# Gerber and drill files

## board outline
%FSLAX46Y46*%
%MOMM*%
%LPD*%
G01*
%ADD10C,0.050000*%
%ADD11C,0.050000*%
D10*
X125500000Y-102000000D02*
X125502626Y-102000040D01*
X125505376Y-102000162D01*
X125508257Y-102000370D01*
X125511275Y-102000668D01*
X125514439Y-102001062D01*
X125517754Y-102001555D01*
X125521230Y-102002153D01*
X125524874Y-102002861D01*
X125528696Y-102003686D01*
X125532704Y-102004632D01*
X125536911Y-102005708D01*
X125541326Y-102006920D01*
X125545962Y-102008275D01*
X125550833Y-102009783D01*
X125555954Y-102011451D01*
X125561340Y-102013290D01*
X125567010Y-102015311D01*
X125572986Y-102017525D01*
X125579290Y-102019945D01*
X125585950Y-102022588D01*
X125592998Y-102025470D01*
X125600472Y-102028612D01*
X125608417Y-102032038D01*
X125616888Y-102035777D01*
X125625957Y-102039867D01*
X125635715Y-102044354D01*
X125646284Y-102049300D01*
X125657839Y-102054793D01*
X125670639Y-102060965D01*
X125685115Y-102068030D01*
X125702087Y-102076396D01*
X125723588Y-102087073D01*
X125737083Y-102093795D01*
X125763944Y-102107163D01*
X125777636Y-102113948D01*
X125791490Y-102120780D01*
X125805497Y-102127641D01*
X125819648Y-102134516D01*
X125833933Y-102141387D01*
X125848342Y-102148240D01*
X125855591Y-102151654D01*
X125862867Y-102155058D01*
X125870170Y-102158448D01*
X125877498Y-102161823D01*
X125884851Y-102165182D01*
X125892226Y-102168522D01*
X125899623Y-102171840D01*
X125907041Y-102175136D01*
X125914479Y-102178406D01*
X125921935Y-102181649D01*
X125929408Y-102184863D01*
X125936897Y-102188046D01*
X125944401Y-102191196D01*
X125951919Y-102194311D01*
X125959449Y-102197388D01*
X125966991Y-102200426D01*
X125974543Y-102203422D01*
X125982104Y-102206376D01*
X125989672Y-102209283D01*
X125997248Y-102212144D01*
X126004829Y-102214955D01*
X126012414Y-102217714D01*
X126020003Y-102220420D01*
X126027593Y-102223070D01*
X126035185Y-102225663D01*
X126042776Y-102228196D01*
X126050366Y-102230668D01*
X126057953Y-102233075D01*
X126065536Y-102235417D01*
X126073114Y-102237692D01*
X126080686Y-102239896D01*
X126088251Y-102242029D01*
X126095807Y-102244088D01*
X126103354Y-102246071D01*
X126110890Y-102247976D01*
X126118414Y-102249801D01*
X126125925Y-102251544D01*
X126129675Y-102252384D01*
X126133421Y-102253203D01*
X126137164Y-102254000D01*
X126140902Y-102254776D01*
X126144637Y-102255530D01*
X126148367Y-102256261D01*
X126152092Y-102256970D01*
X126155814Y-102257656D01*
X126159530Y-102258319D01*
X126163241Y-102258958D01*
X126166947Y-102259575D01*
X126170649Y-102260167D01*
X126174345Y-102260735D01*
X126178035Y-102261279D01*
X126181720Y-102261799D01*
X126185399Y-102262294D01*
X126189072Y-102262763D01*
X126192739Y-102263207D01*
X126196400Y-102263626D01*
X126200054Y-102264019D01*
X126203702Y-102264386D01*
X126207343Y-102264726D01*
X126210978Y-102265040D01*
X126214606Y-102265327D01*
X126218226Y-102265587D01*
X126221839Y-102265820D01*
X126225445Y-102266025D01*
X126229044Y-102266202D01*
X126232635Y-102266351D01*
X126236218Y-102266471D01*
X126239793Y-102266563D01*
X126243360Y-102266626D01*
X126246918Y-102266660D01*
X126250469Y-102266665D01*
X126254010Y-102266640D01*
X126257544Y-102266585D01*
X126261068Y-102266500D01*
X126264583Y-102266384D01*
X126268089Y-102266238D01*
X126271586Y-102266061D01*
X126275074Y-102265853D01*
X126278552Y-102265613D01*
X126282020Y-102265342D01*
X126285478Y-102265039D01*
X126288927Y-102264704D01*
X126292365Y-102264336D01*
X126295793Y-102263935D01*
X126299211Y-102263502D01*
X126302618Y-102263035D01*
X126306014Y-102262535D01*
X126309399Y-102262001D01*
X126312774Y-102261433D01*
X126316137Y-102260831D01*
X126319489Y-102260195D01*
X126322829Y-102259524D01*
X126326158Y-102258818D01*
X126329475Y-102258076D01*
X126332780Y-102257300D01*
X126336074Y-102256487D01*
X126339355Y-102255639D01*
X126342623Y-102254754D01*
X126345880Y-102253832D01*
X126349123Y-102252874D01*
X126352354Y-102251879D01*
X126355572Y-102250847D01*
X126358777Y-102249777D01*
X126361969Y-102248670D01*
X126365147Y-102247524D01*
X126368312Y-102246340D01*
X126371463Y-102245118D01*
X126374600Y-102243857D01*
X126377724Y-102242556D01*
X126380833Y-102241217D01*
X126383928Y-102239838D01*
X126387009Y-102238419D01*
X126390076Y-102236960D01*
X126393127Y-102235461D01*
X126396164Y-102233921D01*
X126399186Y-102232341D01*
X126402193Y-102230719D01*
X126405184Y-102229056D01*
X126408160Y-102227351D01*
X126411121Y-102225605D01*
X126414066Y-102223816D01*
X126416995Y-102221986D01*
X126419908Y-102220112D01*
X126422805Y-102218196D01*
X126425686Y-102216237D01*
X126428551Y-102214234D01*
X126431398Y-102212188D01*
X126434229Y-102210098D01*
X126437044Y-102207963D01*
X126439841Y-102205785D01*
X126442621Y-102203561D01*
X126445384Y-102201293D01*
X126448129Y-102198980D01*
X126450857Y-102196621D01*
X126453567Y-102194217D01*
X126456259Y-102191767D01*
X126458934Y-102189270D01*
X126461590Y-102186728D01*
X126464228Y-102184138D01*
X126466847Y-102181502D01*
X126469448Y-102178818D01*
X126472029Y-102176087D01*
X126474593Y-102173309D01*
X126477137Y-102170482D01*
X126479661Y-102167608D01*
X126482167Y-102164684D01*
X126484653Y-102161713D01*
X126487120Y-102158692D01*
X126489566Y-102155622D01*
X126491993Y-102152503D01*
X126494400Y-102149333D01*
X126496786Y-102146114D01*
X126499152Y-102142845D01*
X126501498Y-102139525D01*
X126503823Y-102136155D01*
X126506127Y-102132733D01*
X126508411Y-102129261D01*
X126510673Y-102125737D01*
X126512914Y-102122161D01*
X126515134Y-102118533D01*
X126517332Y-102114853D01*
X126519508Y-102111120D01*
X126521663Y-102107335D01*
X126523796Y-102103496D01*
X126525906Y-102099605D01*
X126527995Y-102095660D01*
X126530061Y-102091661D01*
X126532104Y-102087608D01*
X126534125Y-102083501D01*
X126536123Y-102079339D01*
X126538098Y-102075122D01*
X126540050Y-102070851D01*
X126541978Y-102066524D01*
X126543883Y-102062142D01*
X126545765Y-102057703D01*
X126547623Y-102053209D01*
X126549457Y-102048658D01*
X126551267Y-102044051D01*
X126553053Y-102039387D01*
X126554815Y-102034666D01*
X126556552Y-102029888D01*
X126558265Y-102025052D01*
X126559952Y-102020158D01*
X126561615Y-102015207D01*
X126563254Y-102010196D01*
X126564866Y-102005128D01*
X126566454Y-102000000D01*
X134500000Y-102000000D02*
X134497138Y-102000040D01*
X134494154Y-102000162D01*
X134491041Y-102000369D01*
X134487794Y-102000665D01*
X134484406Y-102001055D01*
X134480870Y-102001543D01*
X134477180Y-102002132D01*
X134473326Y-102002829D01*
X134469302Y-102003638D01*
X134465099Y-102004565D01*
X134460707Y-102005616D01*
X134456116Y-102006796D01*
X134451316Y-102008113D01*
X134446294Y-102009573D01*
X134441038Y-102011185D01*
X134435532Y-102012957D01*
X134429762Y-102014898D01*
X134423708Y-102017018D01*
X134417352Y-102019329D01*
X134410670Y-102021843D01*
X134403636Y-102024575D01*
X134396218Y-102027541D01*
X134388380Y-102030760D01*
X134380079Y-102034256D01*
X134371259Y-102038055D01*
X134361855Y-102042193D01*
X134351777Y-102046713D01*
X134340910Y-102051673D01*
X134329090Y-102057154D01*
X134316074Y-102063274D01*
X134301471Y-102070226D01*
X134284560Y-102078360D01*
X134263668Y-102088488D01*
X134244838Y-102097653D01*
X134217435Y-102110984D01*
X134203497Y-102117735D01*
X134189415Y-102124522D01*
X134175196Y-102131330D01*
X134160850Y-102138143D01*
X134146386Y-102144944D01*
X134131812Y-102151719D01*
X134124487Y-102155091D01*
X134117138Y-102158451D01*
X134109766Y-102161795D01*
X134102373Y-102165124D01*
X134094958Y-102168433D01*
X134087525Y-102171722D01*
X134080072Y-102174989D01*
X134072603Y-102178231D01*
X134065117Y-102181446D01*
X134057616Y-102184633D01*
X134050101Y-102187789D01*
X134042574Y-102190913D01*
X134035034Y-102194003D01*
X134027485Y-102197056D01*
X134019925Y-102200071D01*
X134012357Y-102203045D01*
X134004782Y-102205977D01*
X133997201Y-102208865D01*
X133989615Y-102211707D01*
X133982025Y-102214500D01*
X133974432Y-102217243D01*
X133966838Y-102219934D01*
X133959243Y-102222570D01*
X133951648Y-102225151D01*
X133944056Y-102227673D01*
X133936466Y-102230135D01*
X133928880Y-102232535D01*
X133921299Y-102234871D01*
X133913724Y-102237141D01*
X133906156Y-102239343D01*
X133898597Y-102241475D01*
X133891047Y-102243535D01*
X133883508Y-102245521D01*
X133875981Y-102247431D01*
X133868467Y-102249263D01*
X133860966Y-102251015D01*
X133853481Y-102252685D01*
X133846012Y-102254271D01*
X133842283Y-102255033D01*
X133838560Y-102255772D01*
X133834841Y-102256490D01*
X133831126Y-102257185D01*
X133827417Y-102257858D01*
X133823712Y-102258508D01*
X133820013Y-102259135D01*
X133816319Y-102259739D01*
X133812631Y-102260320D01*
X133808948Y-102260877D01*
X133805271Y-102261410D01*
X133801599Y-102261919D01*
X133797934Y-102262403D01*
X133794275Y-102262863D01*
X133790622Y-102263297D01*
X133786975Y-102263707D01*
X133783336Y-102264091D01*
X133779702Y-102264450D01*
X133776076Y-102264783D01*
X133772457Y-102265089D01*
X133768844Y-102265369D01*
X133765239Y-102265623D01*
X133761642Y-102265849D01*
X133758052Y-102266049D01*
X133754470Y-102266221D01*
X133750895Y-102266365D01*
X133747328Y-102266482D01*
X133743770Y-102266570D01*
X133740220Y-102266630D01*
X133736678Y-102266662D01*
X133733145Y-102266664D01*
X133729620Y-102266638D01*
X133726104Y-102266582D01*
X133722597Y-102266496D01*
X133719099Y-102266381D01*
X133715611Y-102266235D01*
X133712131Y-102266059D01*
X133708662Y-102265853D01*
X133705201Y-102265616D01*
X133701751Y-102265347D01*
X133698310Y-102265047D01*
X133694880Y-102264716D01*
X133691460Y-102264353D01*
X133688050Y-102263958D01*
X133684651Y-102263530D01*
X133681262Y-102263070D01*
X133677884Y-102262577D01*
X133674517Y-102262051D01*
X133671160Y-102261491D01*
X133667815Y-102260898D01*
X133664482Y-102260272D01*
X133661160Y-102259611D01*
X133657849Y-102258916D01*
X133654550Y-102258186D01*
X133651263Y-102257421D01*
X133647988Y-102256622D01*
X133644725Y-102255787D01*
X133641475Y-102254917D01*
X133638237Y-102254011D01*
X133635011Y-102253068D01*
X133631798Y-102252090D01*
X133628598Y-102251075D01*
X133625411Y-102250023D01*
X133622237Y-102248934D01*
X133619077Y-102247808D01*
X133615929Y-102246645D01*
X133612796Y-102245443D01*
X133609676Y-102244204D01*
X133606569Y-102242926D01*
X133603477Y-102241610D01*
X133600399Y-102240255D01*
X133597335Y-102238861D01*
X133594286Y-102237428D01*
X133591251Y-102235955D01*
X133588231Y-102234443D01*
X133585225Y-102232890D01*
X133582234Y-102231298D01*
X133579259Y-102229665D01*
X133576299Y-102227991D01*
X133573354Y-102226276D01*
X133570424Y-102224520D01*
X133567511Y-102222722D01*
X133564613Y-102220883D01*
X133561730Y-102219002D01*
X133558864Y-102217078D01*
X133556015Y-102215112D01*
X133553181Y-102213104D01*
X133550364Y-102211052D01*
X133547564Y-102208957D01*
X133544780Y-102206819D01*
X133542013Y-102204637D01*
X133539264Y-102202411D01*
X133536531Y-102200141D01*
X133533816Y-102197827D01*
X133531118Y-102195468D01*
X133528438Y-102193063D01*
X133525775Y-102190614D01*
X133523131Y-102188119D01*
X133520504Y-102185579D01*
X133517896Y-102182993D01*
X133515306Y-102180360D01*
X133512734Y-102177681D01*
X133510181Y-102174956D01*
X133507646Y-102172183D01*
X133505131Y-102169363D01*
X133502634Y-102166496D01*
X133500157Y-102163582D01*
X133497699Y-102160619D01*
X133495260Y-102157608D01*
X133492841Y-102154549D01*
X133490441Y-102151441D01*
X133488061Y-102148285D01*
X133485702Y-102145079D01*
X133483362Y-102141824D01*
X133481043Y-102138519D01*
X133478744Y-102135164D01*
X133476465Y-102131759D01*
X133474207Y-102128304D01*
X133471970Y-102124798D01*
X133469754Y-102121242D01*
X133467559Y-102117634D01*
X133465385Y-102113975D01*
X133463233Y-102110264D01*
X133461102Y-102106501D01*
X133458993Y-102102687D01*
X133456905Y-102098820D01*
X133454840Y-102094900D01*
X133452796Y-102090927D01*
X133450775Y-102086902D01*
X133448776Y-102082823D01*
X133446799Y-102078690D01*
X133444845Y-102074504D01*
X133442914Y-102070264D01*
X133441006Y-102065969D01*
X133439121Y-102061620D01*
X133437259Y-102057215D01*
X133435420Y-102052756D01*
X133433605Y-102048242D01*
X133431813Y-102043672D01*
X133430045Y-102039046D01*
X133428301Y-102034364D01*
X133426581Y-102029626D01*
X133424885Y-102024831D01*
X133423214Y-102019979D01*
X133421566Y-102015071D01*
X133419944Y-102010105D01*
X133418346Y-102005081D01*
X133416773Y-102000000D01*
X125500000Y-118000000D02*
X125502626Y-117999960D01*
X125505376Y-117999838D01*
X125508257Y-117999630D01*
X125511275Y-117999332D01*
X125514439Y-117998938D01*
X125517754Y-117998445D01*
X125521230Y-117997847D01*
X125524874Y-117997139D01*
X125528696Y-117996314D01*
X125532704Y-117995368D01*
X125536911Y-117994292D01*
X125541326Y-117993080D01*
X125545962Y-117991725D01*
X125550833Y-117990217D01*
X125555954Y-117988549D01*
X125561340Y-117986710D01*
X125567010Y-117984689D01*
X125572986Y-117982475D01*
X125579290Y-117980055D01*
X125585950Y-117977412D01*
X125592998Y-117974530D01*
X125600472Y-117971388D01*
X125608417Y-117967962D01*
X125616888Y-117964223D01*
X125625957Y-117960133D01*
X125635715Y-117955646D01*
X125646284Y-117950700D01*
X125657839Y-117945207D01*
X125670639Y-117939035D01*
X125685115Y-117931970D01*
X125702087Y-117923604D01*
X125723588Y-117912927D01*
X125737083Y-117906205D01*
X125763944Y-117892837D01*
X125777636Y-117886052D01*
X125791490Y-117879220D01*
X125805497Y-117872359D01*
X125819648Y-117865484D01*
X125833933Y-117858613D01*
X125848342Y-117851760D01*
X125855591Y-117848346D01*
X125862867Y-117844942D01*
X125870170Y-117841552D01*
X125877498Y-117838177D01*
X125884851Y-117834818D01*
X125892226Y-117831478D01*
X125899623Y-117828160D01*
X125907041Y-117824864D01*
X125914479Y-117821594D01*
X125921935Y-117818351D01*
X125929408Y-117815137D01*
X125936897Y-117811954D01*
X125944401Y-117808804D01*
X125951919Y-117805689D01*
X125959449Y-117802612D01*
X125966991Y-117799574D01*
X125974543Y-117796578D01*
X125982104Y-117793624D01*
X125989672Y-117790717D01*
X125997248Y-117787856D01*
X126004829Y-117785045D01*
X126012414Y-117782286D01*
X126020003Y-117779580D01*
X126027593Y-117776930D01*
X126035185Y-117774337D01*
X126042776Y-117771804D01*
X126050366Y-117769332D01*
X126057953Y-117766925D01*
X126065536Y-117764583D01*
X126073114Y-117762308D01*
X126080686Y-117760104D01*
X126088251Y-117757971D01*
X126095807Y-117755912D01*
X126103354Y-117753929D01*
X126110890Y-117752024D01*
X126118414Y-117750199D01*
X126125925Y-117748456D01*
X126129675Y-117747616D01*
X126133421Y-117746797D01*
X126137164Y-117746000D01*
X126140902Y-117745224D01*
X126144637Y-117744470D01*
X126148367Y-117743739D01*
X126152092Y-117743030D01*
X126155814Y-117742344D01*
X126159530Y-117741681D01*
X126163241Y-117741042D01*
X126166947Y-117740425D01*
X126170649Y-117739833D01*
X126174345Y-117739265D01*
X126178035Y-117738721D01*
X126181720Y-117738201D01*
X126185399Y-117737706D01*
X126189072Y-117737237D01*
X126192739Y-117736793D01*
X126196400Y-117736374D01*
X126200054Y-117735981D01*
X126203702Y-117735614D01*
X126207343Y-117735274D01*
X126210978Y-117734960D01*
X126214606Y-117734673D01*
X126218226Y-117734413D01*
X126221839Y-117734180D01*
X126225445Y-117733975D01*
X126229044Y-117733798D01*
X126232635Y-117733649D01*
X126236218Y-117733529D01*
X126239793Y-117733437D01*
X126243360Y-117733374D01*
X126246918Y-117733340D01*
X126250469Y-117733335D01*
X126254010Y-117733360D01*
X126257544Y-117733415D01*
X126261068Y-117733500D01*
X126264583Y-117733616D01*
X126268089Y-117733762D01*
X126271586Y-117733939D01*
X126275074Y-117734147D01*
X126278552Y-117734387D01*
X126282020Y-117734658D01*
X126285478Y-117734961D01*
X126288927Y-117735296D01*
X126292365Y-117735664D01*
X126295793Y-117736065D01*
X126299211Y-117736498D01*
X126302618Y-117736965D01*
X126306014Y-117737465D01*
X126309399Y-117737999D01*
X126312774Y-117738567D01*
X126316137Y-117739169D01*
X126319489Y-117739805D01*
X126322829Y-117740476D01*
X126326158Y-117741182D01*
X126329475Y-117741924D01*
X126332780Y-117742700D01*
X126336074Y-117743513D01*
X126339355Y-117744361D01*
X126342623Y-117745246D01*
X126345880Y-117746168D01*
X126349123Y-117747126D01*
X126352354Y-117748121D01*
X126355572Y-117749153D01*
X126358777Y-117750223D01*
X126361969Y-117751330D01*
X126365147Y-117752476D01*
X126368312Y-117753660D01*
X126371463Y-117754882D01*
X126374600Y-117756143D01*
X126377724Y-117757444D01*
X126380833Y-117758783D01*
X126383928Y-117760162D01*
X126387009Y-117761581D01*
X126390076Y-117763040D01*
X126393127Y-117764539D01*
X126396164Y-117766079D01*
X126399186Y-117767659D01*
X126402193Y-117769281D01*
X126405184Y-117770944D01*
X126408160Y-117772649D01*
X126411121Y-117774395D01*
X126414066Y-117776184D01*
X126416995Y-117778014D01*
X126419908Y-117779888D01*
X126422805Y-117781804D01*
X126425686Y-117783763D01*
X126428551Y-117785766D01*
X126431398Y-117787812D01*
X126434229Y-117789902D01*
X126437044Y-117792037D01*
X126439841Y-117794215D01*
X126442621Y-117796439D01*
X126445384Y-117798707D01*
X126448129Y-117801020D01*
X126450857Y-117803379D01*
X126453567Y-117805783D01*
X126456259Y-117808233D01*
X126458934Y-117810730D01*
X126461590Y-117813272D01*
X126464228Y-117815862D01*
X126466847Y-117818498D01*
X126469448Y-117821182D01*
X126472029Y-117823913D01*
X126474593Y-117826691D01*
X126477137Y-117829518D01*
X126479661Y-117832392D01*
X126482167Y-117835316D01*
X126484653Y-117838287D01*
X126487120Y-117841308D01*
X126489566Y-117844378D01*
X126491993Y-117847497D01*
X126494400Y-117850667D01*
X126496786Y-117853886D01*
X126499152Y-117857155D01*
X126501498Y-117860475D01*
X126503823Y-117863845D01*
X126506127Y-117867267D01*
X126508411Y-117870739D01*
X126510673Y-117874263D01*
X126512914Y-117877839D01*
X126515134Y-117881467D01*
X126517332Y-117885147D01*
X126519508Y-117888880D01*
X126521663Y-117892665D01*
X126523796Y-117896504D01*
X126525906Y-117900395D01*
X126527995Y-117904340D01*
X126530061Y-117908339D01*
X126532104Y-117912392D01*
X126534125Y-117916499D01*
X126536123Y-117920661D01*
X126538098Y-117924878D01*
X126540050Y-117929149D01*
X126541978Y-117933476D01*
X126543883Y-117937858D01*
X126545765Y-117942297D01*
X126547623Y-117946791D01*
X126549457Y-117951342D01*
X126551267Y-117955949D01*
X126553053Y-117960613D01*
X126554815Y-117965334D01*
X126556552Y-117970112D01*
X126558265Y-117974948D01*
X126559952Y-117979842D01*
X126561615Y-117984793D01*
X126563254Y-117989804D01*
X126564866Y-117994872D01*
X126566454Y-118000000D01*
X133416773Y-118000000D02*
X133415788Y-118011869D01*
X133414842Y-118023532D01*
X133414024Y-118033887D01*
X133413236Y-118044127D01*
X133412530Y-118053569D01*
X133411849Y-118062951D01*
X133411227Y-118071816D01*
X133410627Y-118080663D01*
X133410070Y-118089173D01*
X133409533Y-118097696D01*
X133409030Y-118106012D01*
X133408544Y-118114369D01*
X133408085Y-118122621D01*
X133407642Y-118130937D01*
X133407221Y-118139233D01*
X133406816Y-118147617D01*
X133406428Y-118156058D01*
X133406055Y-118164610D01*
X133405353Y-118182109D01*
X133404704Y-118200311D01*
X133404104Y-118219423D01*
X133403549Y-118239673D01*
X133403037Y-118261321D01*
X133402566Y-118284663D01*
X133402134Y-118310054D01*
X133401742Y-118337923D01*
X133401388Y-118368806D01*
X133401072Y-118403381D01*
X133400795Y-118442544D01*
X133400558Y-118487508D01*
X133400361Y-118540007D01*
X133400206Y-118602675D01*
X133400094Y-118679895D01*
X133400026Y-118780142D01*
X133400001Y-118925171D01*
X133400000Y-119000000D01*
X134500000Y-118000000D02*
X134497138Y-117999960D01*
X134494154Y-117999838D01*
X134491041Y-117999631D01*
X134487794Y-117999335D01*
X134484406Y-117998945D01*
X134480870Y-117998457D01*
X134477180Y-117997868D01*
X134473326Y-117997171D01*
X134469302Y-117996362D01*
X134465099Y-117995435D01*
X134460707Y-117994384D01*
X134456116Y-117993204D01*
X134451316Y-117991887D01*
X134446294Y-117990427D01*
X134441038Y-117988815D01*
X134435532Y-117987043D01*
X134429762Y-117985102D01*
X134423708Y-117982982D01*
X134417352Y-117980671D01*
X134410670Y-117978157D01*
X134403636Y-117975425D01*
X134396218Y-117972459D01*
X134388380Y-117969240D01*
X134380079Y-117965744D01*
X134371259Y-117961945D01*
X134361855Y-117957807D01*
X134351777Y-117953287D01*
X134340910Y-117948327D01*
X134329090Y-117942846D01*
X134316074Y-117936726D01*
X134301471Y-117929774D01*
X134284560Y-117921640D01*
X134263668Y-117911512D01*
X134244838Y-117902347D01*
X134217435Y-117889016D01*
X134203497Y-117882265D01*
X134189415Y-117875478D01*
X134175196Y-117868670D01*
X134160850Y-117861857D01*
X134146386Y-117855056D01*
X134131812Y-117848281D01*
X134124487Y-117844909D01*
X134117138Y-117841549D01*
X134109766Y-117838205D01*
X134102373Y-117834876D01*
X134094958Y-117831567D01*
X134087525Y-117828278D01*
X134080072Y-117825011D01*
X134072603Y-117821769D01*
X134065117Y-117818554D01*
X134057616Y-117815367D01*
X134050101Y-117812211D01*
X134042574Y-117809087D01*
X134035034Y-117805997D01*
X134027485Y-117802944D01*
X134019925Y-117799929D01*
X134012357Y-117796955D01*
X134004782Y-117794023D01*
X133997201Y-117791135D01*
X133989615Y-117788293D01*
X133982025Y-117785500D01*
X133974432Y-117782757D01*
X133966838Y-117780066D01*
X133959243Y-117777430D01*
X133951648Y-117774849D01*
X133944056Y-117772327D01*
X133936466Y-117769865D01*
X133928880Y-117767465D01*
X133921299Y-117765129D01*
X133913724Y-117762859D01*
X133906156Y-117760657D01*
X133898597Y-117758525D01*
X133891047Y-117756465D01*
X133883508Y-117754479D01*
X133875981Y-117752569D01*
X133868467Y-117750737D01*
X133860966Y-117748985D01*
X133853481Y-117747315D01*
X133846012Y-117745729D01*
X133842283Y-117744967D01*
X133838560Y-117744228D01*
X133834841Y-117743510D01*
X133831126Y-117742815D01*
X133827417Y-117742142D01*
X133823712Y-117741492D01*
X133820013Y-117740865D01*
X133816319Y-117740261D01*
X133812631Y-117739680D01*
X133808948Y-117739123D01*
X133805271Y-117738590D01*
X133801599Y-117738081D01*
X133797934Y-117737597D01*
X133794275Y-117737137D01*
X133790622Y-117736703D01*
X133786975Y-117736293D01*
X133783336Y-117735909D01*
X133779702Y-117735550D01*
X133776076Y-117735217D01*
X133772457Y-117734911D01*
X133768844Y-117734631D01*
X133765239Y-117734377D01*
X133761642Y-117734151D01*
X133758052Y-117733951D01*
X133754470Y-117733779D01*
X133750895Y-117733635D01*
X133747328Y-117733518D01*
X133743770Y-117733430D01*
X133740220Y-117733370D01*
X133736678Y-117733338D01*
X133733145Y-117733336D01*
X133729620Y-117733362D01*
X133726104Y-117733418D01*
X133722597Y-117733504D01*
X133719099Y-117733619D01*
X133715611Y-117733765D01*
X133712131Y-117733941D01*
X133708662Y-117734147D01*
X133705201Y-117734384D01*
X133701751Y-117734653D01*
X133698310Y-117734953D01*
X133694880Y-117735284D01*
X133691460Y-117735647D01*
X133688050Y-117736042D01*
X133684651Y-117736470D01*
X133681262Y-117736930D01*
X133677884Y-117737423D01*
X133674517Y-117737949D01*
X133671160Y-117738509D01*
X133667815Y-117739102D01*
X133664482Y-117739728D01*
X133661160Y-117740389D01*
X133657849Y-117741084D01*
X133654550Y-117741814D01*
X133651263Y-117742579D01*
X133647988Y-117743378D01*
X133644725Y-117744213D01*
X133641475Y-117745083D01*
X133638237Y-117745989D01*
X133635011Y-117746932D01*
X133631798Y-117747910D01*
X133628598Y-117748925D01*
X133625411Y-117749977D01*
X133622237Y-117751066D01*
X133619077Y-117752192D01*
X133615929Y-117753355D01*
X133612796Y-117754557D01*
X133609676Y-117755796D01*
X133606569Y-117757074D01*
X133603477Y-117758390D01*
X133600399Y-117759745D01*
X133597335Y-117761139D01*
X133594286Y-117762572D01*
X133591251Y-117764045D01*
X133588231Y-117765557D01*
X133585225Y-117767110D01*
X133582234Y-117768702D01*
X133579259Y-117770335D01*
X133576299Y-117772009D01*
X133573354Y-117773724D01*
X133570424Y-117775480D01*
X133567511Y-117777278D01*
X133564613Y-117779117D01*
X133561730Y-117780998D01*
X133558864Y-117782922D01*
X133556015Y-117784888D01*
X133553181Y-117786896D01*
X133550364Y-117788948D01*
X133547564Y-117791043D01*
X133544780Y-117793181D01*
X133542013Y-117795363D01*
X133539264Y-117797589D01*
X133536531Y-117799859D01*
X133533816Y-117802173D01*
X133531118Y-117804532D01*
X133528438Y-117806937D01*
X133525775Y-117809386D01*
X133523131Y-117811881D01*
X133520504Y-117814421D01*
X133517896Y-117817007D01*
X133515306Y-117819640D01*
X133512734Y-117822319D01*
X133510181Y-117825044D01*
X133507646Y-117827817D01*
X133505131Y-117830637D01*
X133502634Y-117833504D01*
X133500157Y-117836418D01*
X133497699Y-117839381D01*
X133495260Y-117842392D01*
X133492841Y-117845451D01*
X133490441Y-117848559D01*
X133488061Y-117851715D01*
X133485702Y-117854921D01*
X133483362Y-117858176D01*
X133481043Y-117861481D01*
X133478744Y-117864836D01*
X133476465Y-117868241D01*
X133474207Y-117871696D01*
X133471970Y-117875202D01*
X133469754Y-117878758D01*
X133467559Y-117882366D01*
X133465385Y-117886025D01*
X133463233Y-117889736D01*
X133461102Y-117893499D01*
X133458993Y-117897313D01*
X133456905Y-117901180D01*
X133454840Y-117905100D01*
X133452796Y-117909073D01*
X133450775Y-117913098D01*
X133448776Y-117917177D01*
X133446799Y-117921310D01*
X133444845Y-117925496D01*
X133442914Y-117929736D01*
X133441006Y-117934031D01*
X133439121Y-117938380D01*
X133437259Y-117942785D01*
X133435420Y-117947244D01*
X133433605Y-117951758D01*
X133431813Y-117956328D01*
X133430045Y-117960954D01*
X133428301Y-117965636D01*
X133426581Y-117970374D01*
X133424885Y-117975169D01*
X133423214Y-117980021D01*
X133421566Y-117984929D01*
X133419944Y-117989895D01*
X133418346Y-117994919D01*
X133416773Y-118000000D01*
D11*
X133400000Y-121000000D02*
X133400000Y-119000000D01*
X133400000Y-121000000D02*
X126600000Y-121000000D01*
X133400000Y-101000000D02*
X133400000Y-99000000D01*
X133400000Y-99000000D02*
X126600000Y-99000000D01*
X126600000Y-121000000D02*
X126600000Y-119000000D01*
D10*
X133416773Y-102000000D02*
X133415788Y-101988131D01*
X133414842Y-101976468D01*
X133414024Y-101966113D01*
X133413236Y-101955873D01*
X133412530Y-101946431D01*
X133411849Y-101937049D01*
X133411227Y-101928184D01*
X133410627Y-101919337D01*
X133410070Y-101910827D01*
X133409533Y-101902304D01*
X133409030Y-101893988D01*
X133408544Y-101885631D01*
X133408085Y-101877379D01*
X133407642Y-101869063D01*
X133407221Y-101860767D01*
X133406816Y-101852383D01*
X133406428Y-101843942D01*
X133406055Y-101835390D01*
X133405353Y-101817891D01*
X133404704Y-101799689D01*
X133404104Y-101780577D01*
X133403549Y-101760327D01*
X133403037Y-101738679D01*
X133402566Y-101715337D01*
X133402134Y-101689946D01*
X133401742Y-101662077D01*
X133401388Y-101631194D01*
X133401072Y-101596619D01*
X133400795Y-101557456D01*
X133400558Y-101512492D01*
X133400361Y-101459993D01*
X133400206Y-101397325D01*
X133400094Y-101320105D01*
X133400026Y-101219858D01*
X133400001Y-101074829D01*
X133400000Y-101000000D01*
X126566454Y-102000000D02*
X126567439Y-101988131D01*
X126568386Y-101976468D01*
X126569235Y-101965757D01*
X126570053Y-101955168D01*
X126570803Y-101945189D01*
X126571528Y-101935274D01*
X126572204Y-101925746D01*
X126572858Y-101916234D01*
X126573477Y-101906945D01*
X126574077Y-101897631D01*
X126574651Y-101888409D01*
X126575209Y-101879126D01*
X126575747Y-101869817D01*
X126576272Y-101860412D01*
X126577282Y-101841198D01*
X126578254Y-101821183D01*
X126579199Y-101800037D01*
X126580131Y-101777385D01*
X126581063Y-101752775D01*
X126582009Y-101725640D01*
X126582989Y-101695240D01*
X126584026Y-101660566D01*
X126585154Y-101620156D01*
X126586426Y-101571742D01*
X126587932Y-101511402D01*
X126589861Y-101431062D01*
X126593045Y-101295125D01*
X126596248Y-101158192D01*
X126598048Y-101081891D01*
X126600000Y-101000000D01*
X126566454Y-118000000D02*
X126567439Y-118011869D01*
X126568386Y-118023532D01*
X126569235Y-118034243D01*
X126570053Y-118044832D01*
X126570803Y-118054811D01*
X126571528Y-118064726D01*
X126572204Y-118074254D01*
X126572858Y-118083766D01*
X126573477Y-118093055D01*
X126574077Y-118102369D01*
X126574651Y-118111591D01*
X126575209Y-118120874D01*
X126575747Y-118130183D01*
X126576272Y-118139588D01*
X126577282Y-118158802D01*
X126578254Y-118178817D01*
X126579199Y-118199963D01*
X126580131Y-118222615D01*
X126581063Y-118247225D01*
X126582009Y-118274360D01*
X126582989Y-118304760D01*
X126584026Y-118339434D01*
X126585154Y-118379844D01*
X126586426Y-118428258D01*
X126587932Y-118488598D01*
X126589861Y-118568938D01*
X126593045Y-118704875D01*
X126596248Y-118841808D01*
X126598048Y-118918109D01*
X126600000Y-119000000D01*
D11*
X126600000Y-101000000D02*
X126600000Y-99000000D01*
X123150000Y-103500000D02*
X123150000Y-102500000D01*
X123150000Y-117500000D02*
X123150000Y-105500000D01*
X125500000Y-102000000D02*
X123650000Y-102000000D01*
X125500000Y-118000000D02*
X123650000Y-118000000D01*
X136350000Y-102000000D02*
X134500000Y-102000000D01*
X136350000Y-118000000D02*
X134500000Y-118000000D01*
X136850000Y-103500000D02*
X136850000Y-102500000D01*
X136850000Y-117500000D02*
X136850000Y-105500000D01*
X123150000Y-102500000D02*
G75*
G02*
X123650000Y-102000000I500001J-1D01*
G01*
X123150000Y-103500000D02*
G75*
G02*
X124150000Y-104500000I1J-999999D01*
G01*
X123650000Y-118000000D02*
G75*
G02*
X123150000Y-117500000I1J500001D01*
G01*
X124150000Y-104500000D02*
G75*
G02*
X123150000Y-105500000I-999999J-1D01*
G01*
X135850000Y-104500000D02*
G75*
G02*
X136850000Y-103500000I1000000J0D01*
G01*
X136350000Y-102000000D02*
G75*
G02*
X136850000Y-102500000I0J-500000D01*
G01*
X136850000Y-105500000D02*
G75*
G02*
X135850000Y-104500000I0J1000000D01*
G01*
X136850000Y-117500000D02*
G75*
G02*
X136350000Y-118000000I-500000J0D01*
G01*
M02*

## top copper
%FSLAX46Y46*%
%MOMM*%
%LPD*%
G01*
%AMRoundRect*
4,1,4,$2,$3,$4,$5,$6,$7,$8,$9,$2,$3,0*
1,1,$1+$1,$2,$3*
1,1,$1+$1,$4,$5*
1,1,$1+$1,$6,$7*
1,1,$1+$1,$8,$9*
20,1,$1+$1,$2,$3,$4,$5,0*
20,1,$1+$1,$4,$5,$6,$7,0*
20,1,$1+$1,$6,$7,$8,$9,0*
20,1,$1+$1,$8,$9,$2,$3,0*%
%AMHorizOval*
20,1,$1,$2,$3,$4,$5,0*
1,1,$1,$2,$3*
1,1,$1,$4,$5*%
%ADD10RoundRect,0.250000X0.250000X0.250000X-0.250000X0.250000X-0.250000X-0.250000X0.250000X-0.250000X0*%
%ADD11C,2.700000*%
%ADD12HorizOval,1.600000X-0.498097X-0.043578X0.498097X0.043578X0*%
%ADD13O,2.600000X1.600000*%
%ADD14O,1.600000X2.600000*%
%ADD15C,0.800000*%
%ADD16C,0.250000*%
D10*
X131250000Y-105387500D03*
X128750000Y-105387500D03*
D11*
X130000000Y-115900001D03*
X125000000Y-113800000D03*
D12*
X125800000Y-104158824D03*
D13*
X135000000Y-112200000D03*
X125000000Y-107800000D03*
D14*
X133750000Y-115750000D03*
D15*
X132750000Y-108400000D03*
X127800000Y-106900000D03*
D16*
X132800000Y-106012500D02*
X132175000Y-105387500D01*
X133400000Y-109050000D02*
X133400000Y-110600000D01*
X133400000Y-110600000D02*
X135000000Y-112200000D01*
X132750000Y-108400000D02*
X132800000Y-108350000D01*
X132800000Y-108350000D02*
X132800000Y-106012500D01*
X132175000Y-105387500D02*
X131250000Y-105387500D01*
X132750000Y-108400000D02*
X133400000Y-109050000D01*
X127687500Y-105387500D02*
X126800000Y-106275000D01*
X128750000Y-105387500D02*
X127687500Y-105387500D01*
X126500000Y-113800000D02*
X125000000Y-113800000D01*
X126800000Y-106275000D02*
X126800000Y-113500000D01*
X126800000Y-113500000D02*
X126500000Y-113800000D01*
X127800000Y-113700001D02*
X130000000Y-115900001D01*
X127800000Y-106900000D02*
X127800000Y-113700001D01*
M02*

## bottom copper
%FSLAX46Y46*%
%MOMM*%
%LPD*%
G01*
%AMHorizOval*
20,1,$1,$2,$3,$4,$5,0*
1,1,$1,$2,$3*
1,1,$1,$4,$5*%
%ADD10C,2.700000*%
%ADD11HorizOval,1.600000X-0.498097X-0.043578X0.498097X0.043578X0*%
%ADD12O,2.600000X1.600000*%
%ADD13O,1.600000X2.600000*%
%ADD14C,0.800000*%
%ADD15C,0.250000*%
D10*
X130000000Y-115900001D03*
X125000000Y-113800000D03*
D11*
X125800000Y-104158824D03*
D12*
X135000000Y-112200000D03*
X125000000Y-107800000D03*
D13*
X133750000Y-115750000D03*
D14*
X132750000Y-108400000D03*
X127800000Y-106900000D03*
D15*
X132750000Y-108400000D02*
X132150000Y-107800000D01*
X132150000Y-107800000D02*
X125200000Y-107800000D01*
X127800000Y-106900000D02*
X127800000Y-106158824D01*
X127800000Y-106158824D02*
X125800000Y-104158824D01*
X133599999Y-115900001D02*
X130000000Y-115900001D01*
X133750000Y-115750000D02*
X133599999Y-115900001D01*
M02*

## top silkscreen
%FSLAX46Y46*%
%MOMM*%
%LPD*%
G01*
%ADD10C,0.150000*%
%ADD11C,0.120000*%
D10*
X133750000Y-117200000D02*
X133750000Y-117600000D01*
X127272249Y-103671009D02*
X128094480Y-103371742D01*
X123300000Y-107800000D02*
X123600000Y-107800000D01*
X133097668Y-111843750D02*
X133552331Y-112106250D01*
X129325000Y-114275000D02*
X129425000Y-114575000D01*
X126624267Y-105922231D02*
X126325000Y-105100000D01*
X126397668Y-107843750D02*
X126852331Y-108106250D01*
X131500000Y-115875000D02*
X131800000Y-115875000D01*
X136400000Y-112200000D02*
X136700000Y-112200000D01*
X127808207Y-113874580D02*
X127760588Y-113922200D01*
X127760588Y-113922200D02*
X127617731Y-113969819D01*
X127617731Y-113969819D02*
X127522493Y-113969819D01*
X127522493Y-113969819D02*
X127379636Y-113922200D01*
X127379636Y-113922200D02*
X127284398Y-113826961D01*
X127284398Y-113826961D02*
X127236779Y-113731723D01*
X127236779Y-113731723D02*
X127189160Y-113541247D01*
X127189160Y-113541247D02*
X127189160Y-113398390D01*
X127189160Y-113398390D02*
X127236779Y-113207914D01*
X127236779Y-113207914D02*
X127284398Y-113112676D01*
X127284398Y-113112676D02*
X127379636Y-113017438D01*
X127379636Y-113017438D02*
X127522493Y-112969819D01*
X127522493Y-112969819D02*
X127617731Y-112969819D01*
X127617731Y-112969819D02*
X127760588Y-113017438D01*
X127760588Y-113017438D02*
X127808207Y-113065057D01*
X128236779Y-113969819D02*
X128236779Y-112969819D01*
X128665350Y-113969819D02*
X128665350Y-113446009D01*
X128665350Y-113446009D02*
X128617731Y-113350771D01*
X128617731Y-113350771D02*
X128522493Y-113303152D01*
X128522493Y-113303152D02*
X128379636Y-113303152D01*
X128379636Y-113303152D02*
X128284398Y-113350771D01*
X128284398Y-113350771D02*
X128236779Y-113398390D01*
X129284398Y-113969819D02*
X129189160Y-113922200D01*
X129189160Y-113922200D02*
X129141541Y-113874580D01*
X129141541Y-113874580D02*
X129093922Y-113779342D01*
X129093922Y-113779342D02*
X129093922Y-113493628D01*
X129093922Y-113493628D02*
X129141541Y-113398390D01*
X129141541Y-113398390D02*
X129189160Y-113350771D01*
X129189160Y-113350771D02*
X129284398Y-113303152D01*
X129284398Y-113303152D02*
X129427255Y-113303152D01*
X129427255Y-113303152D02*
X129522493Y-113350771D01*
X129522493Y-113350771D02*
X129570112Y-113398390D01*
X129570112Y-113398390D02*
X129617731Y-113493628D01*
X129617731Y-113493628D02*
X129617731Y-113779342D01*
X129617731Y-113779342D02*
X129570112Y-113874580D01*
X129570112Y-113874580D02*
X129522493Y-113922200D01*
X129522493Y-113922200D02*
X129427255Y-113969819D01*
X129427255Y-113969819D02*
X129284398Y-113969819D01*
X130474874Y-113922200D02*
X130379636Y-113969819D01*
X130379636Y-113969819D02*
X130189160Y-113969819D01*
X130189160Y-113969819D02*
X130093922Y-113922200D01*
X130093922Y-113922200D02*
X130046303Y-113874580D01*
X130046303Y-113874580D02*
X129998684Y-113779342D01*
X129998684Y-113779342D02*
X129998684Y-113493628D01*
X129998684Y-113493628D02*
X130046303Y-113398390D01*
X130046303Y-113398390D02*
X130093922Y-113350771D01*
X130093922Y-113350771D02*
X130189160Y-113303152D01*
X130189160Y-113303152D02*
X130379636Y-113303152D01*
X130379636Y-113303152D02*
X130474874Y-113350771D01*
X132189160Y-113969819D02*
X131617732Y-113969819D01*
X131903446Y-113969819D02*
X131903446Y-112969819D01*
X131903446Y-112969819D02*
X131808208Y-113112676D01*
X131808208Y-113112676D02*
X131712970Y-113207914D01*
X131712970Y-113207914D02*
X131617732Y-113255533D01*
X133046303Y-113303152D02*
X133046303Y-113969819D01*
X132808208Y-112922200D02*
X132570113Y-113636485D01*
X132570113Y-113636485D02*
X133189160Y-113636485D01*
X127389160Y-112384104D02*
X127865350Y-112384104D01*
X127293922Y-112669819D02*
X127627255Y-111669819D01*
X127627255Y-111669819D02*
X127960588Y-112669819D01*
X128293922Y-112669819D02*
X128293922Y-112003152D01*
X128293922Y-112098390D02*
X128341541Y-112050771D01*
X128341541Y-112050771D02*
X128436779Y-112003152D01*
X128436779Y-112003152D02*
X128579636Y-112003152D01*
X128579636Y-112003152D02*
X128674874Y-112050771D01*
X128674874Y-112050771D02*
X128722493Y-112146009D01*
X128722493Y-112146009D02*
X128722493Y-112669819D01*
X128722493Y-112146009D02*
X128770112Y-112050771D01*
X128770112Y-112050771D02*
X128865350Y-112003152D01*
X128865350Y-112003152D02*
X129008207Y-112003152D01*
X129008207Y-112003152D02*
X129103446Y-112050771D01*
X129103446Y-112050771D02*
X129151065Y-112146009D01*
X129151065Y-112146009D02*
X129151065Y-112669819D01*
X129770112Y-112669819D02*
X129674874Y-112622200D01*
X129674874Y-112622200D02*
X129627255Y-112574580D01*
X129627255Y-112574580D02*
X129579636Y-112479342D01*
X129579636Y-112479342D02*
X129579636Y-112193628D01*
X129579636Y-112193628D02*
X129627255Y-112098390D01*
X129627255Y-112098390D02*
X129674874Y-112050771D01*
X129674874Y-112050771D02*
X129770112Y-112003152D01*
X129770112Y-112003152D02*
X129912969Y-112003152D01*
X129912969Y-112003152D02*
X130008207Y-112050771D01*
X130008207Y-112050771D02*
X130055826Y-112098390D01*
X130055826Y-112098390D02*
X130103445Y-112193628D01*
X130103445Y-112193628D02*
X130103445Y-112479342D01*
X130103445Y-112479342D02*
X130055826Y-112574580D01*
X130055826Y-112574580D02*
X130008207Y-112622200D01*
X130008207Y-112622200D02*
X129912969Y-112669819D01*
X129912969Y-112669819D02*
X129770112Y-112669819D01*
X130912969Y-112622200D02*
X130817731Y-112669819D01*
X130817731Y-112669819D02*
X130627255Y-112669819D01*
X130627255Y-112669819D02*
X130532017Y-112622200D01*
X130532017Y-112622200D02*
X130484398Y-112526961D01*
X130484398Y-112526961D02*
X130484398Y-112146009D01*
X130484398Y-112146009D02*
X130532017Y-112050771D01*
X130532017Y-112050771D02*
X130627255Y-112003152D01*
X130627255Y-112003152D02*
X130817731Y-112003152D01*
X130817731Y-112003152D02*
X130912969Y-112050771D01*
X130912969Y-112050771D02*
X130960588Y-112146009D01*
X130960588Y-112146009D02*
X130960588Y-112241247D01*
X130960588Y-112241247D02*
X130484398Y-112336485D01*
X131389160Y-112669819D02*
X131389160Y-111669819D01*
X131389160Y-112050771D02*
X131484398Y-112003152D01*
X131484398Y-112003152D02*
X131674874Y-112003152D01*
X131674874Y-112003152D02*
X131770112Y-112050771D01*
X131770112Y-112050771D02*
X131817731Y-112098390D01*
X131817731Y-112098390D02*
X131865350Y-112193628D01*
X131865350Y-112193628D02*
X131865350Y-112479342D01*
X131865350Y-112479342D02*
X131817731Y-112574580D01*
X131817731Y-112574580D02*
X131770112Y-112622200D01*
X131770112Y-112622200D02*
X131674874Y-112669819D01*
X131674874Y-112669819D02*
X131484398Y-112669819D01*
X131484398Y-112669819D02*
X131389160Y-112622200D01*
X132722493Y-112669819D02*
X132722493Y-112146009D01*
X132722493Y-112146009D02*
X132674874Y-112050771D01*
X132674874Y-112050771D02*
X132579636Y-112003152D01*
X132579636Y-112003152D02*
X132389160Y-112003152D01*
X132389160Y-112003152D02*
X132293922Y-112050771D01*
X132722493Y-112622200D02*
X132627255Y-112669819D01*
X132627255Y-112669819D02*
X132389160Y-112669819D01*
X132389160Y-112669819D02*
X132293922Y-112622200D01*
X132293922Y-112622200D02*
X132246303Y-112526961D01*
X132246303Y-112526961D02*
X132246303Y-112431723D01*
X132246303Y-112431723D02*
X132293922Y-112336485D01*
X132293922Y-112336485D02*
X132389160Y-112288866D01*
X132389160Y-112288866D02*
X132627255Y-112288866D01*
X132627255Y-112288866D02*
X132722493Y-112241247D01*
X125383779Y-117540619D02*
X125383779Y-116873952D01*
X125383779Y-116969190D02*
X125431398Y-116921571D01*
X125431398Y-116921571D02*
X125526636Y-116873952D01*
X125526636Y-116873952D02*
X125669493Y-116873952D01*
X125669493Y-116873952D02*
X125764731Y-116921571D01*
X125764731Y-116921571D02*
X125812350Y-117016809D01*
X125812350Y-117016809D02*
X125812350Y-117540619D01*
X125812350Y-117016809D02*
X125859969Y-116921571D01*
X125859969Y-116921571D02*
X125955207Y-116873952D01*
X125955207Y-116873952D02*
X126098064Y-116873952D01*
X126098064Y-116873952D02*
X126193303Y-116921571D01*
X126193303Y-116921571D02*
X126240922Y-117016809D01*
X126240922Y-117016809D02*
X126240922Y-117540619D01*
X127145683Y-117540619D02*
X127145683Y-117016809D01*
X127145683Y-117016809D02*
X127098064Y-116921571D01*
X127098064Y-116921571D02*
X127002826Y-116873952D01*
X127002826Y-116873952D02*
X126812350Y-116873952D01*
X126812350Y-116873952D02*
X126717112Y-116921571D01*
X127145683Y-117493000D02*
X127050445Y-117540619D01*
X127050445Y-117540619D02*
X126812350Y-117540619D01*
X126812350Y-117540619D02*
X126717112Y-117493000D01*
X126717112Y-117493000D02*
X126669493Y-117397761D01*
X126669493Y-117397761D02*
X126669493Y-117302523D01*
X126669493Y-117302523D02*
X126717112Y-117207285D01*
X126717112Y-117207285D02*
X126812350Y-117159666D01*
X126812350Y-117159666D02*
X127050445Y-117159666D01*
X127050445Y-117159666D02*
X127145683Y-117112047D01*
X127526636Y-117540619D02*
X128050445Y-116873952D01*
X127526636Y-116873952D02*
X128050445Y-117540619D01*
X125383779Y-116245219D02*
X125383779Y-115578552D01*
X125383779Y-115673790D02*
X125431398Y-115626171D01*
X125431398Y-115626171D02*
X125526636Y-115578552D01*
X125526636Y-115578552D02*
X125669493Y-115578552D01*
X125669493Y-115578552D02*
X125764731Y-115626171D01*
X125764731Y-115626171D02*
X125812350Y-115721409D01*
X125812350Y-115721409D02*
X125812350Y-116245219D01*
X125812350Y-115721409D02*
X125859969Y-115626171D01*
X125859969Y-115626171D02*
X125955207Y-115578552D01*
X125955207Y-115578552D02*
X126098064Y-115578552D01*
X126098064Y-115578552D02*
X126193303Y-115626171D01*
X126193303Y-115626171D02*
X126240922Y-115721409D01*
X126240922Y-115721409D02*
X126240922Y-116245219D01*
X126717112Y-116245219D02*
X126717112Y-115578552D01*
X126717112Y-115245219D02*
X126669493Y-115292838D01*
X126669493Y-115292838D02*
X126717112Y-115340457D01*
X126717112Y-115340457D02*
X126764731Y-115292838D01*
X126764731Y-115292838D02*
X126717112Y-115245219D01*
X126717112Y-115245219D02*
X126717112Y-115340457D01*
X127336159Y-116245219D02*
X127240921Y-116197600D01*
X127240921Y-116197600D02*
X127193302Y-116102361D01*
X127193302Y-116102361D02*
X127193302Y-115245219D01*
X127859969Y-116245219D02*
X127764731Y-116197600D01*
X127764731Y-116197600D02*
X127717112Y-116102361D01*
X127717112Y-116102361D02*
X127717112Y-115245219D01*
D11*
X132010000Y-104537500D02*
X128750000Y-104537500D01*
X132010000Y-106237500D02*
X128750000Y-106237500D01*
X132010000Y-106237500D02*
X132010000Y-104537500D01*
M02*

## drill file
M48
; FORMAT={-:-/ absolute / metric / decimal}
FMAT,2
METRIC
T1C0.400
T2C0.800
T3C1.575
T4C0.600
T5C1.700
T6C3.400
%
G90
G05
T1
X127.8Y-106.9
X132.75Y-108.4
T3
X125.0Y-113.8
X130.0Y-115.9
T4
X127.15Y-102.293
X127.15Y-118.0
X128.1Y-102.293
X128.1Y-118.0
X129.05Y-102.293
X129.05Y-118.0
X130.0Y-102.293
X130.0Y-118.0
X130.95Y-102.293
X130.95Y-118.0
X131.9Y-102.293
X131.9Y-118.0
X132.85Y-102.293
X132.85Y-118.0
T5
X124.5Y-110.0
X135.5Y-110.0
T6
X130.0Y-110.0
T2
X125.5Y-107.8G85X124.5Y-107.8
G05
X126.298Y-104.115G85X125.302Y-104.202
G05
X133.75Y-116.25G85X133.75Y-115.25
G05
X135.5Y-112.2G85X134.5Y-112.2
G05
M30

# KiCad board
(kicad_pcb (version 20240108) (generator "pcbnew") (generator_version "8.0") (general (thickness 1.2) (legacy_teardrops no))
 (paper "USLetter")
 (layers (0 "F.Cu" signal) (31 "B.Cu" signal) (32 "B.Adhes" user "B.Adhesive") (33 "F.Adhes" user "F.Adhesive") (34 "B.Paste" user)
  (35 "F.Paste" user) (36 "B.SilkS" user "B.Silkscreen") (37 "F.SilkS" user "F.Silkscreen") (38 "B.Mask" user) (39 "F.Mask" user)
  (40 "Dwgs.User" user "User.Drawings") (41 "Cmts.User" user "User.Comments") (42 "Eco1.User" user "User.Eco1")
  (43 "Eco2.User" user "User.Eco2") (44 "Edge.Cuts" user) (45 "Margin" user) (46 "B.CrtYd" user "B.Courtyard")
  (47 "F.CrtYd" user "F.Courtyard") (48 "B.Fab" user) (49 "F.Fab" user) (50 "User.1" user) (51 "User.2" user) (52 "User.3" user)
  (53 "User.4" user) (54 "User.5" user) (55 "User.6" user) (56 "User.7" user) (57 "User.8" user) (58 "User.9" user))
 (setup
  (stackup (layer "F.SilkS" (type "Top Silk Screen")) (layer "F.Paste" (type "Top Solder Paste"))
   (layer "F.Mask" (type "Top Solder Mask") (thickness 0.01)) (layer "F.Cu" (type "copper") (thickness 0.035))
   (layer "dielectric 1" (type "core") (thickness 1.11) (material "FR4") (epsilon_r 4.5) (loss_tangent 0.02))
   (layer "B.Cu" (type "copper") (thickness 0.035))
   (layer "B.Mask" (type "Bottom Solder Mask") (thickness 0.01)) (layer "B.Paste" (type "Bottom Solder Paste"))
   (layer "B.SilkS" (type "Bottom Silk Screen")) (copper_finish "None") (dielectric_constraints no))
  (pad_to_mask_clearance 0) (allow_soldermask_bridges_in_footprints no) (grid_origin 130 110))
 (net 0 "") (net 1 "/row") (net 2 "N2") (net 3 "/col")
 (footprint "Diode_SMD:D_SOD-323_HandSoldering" (layer "F.Cu") (at 130 105.3875 180)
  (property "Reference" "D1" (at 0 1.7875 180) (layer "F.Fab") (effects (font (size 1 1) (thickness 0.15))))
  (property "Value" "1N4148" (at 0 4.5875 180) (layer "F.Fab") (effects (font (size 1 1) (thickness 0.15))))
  (fp_line (start -2.01 0.85) (end 1.25 0.85) (stroke (width 0.12) (type solid)) (layer "F.SilkS"))
  (fp_line (start -2.01 -0.85) (end 1.25 -0.85) (stroke (width 0.12) (type solid)) (layer "F.SilkS"))
  (fp_line (start -2.01 -0.85) (end -2.01 0.85) (stroke (width 0.12) (type solid)) (layer "F.SilkS"))
  (pad "1" smd roundrect (at -1.25 0 180) (size 1 1) (layers "F.Cu" "F.Paste" "F.Mask") (roundrect_rratio 0.25) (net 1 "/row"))
  (pad "2" smd roundrect (at 1.25 0 180) (size 1 1) (layers "F.Cu" "F.Paste" "F.Mask") (roundrect_rratio 0.25) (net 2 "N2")))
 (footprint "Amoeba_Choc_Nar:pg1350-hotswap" (layer "F.Cu") (at 130 110)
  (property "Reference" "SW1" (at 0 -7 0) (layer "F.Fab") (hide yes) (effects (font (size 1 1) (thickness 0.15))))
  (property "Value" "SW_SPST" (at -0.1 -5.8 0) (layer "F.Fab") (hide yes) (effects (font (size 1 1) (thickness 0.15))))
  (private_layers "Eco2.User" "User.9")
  (fp_line (start -6.85 -6.5) (end -6.85 -7.5) (stroke (width 0.05) (type solid)) (layer "Edge.Cuts"))
  (fp_line (start -6.85 7.5) (end -6.85 -4.5) (stroke (width 0.05) (type solid)) (layer "Edge.Cuts"))
  (fp_line (start -4.5 -8) (end -6.35 -8) (stroke (width 0.05) (type solid)) (layer "Edge.Cuts"))
  (fp_line (start -4.5 8) (end -6.35 8) (stroke (width 0.05) (type solid)) (layer "Edge.Cuts"))
  (fp_line (start 6.35 -8) (end 4.5 -8) (stroke (width 0.05) (type solid)) (layer "Edge.Cuts"))
  (fp_line (start 6.35 8) (end 4.5 8) (stroke (width 0.05) (type solid)) (layer "Edge.Cuts"))
  (fp_line (start 6.85 -6.5) (end 6.85 -7.5) (stroke (width 0.05) (type solid)) (layer "Edge.Cuts"))
  (fp_line (start 6.85 7.5) (end 6.85 -4.5) (stroke (width 0.05) (type solid)) (layer "Edge.Cuts"))
  (fp_arc (start -6.85 -7.5) (mid -6.703553 -7.853553) (end -6.35 -8) (stroke (width 0.05) (type default)) (layer "Edge.Cuts"))
  (fp_arc (start -6.85 -6.5) (mid -6.142893 -6.207107) (end -5.85 -5.5) (stroke (width 0.05) (type default)) (layer "Edge.Cuts"))
  (fp_arc (start -6.35 8) (mid -6.703553 7.853553) (end -6.85 7.5) (stroke (width 0.05) (type default)) (layer "Edge.Cuts"))
  (fp_arc (start -5.85 -5.5) (mid -6.142893 -4.792893) (end -6.85 -4.5) (stroke (width 0.05) (type default)) (layer "Edge.Cuts"))
  (fp_arc (start 5.85 -5.5) (mid 6.142893 -6.207107) (end 6.85 -6.5) (stroke (width 0.05) (type default)) (layer "Edge.Cuts"))
  (fp_arc (start 6.35 -8) (mid 6.703553 -7.853553) (end 6.85 -7.5) (stroke (width 0.05) (type default)) (layer "Edge.Cuts"))
  (fp_arc (start 6.85 -4.5) (mid 6.142893 -4.792893) (end 5.85 -5.5) (stroke (width 0.05) (type default)) (layer "Edge.Cuts"))
  (fp_arc (start 6.85 7.5) (mid 6.703553 7.853553) (end 6.35 8) (stroke (width 0.05) (type default)) (layer "Edge.Cuts"))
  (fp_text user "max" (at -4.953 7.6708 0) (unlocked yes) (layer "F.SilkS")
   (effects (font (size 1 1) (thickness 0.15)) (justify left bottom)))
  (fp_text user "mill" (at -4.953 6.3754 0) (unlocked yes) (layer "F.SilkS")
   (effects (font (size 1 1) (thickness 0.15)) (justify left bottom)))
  (pad "" np_thru_hole circle (at -5.5 0 180) (size 1.7 1.7) (drill 1.7) (layers "*.Cu" "*.Mask"))
  (pad "" np_thru_hole circle (at 0 0 180) (size 3.4 3.4) (drill 3.4) (layers "*.Cu" "*.Mask"))
  (pad "" np_thru_hole circle (at 5.5 0 180) (size 1.7 1.7) (drill 1.7) (layers "*.Cu" "*.Mask"))
  (pad "1" thru_hole circle (at 0 5.900001 180) (size 2.7 2.7) (drill 1.5748) (layers "*.Cu" "*.Mask") (remove_unused_layers no)
   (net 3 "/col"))
  (pad "2" thru_hole circle (at -5 3.8 180) (size 2.7 2.7) (drill 1.5748) (layers "*.Cu" "*.Mask") (remove_unused_layers no) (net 2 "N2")))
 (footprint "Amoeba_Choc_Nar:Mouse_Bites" (layer "F.Cu") (at 130 118)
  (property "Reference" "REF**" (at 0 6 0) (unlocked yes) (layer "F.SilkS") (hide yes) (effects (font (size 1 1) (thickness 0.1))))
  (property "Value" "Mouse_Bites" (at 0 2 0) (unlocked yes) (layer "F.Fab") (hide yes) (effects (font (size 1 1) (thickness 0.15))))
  (pad "" np_thru_hole circle (at -2.85 0) (size 0.6 0.6) (drill 0.6) (layers "*.Mask"))
  (pad "" np_thru_hole circle (at -1.9 0) (size 0.6 0.6) (drill 0.6) (layers "*.Mask"))
  (pad "" np_thru_hole circle (at -0.95 0) (size 0.6 0.6) (drill 0.6) (layers "*.Mask"))
  (pad "" np_thru_hole circle (at 0 0) (size 0.6 0.6) (drill 0.6) (layers "*.Mask"))
  (pad "" np_thru_hole circle (at 0.95 0) (size 0.6 0.6) (drill 0.6) (layers "*.Mask"))
  (pad "" np_thru_hole circle (at 1.9 0) (size 0.6 0.6) (drill 0.6) (layers "*.Mask"))
  (pad "" np_thru_hole circle (at 2.85 0) (size 0.6 0.6) (drill 0.6) (layers "*.Mask")))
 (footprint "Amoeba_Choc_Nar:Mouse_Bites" (layer "F.Cu") (at 130 102.292893)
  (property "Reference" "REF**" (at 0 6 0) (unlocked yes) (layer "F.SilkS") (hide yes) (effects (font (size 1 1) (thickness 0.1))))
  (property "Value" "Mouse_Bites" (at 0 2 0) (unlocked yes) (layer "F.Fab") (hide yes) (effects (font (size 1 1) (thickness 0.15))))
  (pad "" np_thru_hole circle (at -2.85 0) (size 0.6 0.6) (drill 0.6) (layers "*.Mask"))
  (pad "" np_thru_hole circle (at -1.9 0) (size 0.6 0.6) (drill 0.6) (layers "*.Mask"))
  (pad "" np_thru_hole circle (at -0.95 0) (size 0.6 0.6) (drill 0.6) (layers "*.Mask"))
  (pad "" np_thru_hole circle (at 0 0) (size 0.6 0.6) (drill 0.6) (layers "*.Mask"))
  (pad "" np_thru_hole circle (at 0.95 0) (size 0.6 0.6) (drill 0.6) (layers "*.Mask"))
  (pad "" np_thru_hole circle (at 1.9 0) (size 0.6 0.6) (drill 0.6) (layers "*.Mask"))
  (pad "" np_thru_hole circle (at 2.85 0) (size 0.6 0.6) (drill 0.6) (layers "*.Mask")))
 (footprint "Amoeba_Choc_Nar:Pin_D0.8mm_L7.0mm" (layer "B.Cu") (at 125.8 104.158824 -85)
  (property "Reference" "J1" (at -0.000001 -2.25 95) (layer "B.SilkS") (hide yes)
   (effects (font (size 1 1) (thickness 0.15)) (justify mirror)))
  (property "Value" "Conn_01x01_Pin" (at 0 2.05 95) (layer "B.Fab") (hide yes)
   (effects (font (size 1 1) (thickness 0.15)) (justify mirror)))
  (pad "1" thru_hole oval (at 0 0 275) (size 1.6 2.6) (drill oval 0.8 1.8) (layers "*.Cu" "*.Mask") (remove_unused_layers no) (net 3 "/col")))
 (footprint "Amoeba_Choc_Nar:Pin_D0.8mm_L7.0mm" (layer "B.Cu") (at 135 112.2 -90)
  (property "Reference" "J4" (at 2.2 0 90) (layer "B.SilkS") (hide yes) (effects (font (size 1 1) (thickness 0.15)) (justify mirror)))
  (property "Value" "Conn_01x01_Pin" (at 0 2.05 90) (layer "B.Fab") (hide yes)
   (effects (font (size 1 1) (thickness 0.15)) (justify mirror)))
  (pad "1" thru_hole oval (at 0 0 270) (size 1.6 2.6) (drill oval 0.8 1.8) (layers "*.Cu" "*.Mask") (remove_unused_layers no) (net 1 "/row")))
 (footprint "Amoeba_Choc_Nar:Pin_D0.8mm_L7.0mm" (layer "B.Cu") (at 125 107.8 -90)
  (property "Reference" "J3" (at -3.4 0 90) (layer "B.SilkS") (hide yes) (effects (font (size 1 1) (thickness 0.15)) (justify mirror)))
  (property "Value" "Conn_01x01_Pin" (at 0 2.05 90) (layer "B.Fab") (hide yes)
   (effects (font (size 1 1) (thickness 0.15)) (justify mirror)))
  (pad "1" thru_hole oval (at 0 0 270) (size 1.6 2.6) (drill oval 0.8 1.8) (layers "*.Cu" "*.Mask") (remove_unused_layers no) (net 1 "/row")))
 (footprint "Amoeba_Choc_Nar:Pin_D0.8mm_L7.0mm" (layer "B.Cu") (at 133.75 115.75 180)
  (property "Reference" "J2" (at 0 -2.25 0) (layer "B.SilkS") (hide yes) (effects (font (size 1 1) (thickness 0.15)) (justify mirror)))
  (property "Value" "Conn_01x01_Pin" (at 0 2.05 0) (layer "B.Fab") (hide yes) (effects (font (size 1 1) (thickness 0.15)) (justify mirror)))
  (pad "1" thru_hole oval (at 0 0 180) (size 1.6 2.6) (drill oval 0.8 1.8) (layers "*.Cu" "*.Mask") (remove_unused_layers no) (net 3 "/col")))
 (gr_line (start 133.75 117.2) (end 133.75 117.6) (stroke (width 0.15) (type default)) (layer "F.SilkS"))
 (gr_line (start 127.272249 103.671009) (end 128.09448 103.371742) (stroke (width 0.15) (type default)) (layer "F.SilkS"))
 (gr_line (start 123.3 107.8) (end 123.6 107.8) (stroke (width 0.15) (type default)) (layer "F.SilkS"))
 (gr_line (start 133.097668 111.84375) (end 133.552331 112.10625) (stroke (width 0.15) (type default)) (layer "F.SilkS"))
 (gr_line (start 129.325 114.275) (end 129.425 114.575) (stroke (width 0.15) (type default)) (layer "F.SilkS"))
 (gr_line (start 126.624267 105.922231) (end 126.325 105.1) (stroke (width 0.15) (type default)) (layer "F.SilkS"))
 (gr_line (start 126.397668 107.84375) (end 126.852331 108.10625) (stroke (width 0.15) (type default)) (layer "F.SilkS"))
 (gr_line (start 131.5 115.875) (end 131.8 115.875) (stroke (width 0.15) (type default)) (layer "F.SilkS"))
 (gr_line (start 136.4 112.2) (end 136.7 112.2) (stroke (width 0.15) (type default)) (layer "F.SilkS"))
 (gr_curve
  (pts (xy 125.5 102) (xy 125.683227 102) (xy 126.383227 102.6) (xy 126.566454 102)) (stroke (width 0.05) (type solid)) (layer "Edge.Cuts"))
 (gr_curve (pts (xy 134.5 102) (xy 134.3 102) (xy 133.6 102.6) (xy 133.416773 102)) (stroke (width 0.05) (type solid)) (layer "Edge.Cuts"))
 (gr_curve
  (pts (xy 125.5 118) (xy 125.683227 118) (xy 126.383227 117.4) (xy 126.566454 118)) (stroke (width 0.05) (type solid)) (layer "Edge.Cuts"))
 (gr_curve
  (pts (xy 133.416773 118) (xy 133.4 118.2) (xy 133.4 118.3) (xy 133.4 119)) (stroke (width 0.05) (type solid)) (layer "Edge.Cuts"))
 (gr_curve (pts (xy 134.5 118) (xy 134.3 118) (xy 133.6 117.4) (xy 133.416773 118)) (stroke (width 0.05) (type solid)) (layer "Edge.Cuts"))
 (gr_line (start 133.4 121) (end 133.4 119) (stroke (width 0.05) (type default)) (layer "Edge.Cuts"))
 (gr_line (start 133.4 121) (end 126.6 121) (stroke (width 0.05) (type default)) (layer "Edge.Cuts"))
 (gr_line (start 133.4 101) (end 133.4 99) (stroke (width 0.05) (type default)) (layer "Edge.Cuts"))
 (gr_line (start 133.4 99) (end 126.6 99) (stroke (width 0.05) (type default)) (layer "Edge.Cuts"))
 (gr_line (start 126.6 121) (end 126.6 119) (stroke (width 0.05) (type default)) (layer "Edge.Cuts"))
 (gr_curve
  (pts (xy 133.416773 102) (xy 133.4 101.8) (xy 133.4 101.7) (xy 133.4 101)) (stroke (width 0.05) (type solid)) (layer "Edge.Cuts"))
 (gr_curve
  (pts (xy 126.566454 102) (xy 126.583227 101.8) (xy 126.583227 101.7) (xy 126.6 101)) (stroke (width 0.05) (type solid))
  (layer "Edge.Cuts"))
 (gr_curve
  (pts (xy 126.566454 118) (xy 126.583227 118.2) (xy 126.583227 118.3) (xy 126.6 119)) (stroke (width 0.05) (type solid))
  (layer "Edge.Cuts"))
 (gr_line (start 126.6 101) (end 126.6 99) (stroke (width 0.05) (type default)) (layer "Edge.Cuts"))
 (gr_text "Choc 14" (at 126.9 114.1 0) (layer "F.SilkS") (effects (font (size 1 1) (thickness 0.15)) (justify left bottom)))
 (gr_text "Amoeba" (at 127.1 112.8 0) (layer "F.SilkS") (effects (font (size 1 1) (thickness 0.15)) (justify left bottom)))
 (segment (start 132.8 106.0125) (end 132.175 105.3875) (width 0.25) (layer "F.Cu") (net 1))
 (segment (start 133.4 109.05) (end 133.4 110.6) (width 0.25) (layer "F.Cu") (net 1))
 (segment (start 133.4 110.6) (end 135 112.2) (width 0.25) (layer "F.Cu") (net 1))
 (segment (start 132.75 108.4) (end 132.8 108.35) (width 0.25) (layer "F.Cu") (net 1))
 (segment (start 132.8 108.35) (end 132.8 106.0125) (width 0.25) (layer "F.Cu") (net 1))
 (segment (start 132.175 105.3875) (end 131.25 105.3875) (width 0.25) (layer "F.Cu") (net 1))
 (segment (start 132.75 108.4) (end 133.4 109.05) (width 0.25) (layer "F.Cu") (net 1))
 (via (at 132.75 108.4) (size 0.8) (drill 0.4) (layers "F.Cu" "B.Cu") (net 1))
 (segment (start 132.75 108.4) (end 132.15 107.8) (width 0.25) (layer "B.Cu") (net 1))
 (segment (start 132.15 107.8) (end 125.2 107.8) (width 0.25) (layer "B.Cu") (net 1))
 (segment (start 127.6875 105.3875) (end 126.8 106.275) (width 0.25) (layer "F.Cu") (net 2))
 (segment (start 128.75 105.3875) (end 127.6875 105.3875) (width 0.25) (layer "F.Cu") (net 2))
 (segment (start 126.5 113.8) (end 125 113.8) (width 0.25) (layer "F.Cu") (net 2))
 (segment (start 126.8 106.275) (end 126.8 113.5) (width 0.25) (layer "F.Cu") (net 2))
 (segment (start 126.8 113.5) (end 126.5 113.8) (width 0.25) (layer "F.Cu") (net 2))
 (segment (start 127.8 113.700001) (end 130 115.900001) (width 0.25) (layer "F.Cu") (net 3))
 (segment (start 127.8 106.9) (end 127.8 113.700001) (width 0.25) (layer "F.Cu") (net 3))
 (via (at 127.8 106.9) (size 0.8) (drill 0.4) (layers "F.Cu" "B.Cu") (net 3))
 (segment (start 127.8 106.9) (end 127.8 106.158824) (width 0.25) (layer "B.Cu") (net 3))
 (segment (start 127.8 106.158824) (end 125.8 104.158824) (width 0.25) (layer "B.Cu") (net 3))
 (segment (start 133.599999 115.900001) (end 130 115.900001) (width 0.25) (layer "B.Cu") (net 3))
 (segment (start 133.75 115.75) (end 133.599999 115.900001) (width 0.25) (layer "B.Cu") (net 3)))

